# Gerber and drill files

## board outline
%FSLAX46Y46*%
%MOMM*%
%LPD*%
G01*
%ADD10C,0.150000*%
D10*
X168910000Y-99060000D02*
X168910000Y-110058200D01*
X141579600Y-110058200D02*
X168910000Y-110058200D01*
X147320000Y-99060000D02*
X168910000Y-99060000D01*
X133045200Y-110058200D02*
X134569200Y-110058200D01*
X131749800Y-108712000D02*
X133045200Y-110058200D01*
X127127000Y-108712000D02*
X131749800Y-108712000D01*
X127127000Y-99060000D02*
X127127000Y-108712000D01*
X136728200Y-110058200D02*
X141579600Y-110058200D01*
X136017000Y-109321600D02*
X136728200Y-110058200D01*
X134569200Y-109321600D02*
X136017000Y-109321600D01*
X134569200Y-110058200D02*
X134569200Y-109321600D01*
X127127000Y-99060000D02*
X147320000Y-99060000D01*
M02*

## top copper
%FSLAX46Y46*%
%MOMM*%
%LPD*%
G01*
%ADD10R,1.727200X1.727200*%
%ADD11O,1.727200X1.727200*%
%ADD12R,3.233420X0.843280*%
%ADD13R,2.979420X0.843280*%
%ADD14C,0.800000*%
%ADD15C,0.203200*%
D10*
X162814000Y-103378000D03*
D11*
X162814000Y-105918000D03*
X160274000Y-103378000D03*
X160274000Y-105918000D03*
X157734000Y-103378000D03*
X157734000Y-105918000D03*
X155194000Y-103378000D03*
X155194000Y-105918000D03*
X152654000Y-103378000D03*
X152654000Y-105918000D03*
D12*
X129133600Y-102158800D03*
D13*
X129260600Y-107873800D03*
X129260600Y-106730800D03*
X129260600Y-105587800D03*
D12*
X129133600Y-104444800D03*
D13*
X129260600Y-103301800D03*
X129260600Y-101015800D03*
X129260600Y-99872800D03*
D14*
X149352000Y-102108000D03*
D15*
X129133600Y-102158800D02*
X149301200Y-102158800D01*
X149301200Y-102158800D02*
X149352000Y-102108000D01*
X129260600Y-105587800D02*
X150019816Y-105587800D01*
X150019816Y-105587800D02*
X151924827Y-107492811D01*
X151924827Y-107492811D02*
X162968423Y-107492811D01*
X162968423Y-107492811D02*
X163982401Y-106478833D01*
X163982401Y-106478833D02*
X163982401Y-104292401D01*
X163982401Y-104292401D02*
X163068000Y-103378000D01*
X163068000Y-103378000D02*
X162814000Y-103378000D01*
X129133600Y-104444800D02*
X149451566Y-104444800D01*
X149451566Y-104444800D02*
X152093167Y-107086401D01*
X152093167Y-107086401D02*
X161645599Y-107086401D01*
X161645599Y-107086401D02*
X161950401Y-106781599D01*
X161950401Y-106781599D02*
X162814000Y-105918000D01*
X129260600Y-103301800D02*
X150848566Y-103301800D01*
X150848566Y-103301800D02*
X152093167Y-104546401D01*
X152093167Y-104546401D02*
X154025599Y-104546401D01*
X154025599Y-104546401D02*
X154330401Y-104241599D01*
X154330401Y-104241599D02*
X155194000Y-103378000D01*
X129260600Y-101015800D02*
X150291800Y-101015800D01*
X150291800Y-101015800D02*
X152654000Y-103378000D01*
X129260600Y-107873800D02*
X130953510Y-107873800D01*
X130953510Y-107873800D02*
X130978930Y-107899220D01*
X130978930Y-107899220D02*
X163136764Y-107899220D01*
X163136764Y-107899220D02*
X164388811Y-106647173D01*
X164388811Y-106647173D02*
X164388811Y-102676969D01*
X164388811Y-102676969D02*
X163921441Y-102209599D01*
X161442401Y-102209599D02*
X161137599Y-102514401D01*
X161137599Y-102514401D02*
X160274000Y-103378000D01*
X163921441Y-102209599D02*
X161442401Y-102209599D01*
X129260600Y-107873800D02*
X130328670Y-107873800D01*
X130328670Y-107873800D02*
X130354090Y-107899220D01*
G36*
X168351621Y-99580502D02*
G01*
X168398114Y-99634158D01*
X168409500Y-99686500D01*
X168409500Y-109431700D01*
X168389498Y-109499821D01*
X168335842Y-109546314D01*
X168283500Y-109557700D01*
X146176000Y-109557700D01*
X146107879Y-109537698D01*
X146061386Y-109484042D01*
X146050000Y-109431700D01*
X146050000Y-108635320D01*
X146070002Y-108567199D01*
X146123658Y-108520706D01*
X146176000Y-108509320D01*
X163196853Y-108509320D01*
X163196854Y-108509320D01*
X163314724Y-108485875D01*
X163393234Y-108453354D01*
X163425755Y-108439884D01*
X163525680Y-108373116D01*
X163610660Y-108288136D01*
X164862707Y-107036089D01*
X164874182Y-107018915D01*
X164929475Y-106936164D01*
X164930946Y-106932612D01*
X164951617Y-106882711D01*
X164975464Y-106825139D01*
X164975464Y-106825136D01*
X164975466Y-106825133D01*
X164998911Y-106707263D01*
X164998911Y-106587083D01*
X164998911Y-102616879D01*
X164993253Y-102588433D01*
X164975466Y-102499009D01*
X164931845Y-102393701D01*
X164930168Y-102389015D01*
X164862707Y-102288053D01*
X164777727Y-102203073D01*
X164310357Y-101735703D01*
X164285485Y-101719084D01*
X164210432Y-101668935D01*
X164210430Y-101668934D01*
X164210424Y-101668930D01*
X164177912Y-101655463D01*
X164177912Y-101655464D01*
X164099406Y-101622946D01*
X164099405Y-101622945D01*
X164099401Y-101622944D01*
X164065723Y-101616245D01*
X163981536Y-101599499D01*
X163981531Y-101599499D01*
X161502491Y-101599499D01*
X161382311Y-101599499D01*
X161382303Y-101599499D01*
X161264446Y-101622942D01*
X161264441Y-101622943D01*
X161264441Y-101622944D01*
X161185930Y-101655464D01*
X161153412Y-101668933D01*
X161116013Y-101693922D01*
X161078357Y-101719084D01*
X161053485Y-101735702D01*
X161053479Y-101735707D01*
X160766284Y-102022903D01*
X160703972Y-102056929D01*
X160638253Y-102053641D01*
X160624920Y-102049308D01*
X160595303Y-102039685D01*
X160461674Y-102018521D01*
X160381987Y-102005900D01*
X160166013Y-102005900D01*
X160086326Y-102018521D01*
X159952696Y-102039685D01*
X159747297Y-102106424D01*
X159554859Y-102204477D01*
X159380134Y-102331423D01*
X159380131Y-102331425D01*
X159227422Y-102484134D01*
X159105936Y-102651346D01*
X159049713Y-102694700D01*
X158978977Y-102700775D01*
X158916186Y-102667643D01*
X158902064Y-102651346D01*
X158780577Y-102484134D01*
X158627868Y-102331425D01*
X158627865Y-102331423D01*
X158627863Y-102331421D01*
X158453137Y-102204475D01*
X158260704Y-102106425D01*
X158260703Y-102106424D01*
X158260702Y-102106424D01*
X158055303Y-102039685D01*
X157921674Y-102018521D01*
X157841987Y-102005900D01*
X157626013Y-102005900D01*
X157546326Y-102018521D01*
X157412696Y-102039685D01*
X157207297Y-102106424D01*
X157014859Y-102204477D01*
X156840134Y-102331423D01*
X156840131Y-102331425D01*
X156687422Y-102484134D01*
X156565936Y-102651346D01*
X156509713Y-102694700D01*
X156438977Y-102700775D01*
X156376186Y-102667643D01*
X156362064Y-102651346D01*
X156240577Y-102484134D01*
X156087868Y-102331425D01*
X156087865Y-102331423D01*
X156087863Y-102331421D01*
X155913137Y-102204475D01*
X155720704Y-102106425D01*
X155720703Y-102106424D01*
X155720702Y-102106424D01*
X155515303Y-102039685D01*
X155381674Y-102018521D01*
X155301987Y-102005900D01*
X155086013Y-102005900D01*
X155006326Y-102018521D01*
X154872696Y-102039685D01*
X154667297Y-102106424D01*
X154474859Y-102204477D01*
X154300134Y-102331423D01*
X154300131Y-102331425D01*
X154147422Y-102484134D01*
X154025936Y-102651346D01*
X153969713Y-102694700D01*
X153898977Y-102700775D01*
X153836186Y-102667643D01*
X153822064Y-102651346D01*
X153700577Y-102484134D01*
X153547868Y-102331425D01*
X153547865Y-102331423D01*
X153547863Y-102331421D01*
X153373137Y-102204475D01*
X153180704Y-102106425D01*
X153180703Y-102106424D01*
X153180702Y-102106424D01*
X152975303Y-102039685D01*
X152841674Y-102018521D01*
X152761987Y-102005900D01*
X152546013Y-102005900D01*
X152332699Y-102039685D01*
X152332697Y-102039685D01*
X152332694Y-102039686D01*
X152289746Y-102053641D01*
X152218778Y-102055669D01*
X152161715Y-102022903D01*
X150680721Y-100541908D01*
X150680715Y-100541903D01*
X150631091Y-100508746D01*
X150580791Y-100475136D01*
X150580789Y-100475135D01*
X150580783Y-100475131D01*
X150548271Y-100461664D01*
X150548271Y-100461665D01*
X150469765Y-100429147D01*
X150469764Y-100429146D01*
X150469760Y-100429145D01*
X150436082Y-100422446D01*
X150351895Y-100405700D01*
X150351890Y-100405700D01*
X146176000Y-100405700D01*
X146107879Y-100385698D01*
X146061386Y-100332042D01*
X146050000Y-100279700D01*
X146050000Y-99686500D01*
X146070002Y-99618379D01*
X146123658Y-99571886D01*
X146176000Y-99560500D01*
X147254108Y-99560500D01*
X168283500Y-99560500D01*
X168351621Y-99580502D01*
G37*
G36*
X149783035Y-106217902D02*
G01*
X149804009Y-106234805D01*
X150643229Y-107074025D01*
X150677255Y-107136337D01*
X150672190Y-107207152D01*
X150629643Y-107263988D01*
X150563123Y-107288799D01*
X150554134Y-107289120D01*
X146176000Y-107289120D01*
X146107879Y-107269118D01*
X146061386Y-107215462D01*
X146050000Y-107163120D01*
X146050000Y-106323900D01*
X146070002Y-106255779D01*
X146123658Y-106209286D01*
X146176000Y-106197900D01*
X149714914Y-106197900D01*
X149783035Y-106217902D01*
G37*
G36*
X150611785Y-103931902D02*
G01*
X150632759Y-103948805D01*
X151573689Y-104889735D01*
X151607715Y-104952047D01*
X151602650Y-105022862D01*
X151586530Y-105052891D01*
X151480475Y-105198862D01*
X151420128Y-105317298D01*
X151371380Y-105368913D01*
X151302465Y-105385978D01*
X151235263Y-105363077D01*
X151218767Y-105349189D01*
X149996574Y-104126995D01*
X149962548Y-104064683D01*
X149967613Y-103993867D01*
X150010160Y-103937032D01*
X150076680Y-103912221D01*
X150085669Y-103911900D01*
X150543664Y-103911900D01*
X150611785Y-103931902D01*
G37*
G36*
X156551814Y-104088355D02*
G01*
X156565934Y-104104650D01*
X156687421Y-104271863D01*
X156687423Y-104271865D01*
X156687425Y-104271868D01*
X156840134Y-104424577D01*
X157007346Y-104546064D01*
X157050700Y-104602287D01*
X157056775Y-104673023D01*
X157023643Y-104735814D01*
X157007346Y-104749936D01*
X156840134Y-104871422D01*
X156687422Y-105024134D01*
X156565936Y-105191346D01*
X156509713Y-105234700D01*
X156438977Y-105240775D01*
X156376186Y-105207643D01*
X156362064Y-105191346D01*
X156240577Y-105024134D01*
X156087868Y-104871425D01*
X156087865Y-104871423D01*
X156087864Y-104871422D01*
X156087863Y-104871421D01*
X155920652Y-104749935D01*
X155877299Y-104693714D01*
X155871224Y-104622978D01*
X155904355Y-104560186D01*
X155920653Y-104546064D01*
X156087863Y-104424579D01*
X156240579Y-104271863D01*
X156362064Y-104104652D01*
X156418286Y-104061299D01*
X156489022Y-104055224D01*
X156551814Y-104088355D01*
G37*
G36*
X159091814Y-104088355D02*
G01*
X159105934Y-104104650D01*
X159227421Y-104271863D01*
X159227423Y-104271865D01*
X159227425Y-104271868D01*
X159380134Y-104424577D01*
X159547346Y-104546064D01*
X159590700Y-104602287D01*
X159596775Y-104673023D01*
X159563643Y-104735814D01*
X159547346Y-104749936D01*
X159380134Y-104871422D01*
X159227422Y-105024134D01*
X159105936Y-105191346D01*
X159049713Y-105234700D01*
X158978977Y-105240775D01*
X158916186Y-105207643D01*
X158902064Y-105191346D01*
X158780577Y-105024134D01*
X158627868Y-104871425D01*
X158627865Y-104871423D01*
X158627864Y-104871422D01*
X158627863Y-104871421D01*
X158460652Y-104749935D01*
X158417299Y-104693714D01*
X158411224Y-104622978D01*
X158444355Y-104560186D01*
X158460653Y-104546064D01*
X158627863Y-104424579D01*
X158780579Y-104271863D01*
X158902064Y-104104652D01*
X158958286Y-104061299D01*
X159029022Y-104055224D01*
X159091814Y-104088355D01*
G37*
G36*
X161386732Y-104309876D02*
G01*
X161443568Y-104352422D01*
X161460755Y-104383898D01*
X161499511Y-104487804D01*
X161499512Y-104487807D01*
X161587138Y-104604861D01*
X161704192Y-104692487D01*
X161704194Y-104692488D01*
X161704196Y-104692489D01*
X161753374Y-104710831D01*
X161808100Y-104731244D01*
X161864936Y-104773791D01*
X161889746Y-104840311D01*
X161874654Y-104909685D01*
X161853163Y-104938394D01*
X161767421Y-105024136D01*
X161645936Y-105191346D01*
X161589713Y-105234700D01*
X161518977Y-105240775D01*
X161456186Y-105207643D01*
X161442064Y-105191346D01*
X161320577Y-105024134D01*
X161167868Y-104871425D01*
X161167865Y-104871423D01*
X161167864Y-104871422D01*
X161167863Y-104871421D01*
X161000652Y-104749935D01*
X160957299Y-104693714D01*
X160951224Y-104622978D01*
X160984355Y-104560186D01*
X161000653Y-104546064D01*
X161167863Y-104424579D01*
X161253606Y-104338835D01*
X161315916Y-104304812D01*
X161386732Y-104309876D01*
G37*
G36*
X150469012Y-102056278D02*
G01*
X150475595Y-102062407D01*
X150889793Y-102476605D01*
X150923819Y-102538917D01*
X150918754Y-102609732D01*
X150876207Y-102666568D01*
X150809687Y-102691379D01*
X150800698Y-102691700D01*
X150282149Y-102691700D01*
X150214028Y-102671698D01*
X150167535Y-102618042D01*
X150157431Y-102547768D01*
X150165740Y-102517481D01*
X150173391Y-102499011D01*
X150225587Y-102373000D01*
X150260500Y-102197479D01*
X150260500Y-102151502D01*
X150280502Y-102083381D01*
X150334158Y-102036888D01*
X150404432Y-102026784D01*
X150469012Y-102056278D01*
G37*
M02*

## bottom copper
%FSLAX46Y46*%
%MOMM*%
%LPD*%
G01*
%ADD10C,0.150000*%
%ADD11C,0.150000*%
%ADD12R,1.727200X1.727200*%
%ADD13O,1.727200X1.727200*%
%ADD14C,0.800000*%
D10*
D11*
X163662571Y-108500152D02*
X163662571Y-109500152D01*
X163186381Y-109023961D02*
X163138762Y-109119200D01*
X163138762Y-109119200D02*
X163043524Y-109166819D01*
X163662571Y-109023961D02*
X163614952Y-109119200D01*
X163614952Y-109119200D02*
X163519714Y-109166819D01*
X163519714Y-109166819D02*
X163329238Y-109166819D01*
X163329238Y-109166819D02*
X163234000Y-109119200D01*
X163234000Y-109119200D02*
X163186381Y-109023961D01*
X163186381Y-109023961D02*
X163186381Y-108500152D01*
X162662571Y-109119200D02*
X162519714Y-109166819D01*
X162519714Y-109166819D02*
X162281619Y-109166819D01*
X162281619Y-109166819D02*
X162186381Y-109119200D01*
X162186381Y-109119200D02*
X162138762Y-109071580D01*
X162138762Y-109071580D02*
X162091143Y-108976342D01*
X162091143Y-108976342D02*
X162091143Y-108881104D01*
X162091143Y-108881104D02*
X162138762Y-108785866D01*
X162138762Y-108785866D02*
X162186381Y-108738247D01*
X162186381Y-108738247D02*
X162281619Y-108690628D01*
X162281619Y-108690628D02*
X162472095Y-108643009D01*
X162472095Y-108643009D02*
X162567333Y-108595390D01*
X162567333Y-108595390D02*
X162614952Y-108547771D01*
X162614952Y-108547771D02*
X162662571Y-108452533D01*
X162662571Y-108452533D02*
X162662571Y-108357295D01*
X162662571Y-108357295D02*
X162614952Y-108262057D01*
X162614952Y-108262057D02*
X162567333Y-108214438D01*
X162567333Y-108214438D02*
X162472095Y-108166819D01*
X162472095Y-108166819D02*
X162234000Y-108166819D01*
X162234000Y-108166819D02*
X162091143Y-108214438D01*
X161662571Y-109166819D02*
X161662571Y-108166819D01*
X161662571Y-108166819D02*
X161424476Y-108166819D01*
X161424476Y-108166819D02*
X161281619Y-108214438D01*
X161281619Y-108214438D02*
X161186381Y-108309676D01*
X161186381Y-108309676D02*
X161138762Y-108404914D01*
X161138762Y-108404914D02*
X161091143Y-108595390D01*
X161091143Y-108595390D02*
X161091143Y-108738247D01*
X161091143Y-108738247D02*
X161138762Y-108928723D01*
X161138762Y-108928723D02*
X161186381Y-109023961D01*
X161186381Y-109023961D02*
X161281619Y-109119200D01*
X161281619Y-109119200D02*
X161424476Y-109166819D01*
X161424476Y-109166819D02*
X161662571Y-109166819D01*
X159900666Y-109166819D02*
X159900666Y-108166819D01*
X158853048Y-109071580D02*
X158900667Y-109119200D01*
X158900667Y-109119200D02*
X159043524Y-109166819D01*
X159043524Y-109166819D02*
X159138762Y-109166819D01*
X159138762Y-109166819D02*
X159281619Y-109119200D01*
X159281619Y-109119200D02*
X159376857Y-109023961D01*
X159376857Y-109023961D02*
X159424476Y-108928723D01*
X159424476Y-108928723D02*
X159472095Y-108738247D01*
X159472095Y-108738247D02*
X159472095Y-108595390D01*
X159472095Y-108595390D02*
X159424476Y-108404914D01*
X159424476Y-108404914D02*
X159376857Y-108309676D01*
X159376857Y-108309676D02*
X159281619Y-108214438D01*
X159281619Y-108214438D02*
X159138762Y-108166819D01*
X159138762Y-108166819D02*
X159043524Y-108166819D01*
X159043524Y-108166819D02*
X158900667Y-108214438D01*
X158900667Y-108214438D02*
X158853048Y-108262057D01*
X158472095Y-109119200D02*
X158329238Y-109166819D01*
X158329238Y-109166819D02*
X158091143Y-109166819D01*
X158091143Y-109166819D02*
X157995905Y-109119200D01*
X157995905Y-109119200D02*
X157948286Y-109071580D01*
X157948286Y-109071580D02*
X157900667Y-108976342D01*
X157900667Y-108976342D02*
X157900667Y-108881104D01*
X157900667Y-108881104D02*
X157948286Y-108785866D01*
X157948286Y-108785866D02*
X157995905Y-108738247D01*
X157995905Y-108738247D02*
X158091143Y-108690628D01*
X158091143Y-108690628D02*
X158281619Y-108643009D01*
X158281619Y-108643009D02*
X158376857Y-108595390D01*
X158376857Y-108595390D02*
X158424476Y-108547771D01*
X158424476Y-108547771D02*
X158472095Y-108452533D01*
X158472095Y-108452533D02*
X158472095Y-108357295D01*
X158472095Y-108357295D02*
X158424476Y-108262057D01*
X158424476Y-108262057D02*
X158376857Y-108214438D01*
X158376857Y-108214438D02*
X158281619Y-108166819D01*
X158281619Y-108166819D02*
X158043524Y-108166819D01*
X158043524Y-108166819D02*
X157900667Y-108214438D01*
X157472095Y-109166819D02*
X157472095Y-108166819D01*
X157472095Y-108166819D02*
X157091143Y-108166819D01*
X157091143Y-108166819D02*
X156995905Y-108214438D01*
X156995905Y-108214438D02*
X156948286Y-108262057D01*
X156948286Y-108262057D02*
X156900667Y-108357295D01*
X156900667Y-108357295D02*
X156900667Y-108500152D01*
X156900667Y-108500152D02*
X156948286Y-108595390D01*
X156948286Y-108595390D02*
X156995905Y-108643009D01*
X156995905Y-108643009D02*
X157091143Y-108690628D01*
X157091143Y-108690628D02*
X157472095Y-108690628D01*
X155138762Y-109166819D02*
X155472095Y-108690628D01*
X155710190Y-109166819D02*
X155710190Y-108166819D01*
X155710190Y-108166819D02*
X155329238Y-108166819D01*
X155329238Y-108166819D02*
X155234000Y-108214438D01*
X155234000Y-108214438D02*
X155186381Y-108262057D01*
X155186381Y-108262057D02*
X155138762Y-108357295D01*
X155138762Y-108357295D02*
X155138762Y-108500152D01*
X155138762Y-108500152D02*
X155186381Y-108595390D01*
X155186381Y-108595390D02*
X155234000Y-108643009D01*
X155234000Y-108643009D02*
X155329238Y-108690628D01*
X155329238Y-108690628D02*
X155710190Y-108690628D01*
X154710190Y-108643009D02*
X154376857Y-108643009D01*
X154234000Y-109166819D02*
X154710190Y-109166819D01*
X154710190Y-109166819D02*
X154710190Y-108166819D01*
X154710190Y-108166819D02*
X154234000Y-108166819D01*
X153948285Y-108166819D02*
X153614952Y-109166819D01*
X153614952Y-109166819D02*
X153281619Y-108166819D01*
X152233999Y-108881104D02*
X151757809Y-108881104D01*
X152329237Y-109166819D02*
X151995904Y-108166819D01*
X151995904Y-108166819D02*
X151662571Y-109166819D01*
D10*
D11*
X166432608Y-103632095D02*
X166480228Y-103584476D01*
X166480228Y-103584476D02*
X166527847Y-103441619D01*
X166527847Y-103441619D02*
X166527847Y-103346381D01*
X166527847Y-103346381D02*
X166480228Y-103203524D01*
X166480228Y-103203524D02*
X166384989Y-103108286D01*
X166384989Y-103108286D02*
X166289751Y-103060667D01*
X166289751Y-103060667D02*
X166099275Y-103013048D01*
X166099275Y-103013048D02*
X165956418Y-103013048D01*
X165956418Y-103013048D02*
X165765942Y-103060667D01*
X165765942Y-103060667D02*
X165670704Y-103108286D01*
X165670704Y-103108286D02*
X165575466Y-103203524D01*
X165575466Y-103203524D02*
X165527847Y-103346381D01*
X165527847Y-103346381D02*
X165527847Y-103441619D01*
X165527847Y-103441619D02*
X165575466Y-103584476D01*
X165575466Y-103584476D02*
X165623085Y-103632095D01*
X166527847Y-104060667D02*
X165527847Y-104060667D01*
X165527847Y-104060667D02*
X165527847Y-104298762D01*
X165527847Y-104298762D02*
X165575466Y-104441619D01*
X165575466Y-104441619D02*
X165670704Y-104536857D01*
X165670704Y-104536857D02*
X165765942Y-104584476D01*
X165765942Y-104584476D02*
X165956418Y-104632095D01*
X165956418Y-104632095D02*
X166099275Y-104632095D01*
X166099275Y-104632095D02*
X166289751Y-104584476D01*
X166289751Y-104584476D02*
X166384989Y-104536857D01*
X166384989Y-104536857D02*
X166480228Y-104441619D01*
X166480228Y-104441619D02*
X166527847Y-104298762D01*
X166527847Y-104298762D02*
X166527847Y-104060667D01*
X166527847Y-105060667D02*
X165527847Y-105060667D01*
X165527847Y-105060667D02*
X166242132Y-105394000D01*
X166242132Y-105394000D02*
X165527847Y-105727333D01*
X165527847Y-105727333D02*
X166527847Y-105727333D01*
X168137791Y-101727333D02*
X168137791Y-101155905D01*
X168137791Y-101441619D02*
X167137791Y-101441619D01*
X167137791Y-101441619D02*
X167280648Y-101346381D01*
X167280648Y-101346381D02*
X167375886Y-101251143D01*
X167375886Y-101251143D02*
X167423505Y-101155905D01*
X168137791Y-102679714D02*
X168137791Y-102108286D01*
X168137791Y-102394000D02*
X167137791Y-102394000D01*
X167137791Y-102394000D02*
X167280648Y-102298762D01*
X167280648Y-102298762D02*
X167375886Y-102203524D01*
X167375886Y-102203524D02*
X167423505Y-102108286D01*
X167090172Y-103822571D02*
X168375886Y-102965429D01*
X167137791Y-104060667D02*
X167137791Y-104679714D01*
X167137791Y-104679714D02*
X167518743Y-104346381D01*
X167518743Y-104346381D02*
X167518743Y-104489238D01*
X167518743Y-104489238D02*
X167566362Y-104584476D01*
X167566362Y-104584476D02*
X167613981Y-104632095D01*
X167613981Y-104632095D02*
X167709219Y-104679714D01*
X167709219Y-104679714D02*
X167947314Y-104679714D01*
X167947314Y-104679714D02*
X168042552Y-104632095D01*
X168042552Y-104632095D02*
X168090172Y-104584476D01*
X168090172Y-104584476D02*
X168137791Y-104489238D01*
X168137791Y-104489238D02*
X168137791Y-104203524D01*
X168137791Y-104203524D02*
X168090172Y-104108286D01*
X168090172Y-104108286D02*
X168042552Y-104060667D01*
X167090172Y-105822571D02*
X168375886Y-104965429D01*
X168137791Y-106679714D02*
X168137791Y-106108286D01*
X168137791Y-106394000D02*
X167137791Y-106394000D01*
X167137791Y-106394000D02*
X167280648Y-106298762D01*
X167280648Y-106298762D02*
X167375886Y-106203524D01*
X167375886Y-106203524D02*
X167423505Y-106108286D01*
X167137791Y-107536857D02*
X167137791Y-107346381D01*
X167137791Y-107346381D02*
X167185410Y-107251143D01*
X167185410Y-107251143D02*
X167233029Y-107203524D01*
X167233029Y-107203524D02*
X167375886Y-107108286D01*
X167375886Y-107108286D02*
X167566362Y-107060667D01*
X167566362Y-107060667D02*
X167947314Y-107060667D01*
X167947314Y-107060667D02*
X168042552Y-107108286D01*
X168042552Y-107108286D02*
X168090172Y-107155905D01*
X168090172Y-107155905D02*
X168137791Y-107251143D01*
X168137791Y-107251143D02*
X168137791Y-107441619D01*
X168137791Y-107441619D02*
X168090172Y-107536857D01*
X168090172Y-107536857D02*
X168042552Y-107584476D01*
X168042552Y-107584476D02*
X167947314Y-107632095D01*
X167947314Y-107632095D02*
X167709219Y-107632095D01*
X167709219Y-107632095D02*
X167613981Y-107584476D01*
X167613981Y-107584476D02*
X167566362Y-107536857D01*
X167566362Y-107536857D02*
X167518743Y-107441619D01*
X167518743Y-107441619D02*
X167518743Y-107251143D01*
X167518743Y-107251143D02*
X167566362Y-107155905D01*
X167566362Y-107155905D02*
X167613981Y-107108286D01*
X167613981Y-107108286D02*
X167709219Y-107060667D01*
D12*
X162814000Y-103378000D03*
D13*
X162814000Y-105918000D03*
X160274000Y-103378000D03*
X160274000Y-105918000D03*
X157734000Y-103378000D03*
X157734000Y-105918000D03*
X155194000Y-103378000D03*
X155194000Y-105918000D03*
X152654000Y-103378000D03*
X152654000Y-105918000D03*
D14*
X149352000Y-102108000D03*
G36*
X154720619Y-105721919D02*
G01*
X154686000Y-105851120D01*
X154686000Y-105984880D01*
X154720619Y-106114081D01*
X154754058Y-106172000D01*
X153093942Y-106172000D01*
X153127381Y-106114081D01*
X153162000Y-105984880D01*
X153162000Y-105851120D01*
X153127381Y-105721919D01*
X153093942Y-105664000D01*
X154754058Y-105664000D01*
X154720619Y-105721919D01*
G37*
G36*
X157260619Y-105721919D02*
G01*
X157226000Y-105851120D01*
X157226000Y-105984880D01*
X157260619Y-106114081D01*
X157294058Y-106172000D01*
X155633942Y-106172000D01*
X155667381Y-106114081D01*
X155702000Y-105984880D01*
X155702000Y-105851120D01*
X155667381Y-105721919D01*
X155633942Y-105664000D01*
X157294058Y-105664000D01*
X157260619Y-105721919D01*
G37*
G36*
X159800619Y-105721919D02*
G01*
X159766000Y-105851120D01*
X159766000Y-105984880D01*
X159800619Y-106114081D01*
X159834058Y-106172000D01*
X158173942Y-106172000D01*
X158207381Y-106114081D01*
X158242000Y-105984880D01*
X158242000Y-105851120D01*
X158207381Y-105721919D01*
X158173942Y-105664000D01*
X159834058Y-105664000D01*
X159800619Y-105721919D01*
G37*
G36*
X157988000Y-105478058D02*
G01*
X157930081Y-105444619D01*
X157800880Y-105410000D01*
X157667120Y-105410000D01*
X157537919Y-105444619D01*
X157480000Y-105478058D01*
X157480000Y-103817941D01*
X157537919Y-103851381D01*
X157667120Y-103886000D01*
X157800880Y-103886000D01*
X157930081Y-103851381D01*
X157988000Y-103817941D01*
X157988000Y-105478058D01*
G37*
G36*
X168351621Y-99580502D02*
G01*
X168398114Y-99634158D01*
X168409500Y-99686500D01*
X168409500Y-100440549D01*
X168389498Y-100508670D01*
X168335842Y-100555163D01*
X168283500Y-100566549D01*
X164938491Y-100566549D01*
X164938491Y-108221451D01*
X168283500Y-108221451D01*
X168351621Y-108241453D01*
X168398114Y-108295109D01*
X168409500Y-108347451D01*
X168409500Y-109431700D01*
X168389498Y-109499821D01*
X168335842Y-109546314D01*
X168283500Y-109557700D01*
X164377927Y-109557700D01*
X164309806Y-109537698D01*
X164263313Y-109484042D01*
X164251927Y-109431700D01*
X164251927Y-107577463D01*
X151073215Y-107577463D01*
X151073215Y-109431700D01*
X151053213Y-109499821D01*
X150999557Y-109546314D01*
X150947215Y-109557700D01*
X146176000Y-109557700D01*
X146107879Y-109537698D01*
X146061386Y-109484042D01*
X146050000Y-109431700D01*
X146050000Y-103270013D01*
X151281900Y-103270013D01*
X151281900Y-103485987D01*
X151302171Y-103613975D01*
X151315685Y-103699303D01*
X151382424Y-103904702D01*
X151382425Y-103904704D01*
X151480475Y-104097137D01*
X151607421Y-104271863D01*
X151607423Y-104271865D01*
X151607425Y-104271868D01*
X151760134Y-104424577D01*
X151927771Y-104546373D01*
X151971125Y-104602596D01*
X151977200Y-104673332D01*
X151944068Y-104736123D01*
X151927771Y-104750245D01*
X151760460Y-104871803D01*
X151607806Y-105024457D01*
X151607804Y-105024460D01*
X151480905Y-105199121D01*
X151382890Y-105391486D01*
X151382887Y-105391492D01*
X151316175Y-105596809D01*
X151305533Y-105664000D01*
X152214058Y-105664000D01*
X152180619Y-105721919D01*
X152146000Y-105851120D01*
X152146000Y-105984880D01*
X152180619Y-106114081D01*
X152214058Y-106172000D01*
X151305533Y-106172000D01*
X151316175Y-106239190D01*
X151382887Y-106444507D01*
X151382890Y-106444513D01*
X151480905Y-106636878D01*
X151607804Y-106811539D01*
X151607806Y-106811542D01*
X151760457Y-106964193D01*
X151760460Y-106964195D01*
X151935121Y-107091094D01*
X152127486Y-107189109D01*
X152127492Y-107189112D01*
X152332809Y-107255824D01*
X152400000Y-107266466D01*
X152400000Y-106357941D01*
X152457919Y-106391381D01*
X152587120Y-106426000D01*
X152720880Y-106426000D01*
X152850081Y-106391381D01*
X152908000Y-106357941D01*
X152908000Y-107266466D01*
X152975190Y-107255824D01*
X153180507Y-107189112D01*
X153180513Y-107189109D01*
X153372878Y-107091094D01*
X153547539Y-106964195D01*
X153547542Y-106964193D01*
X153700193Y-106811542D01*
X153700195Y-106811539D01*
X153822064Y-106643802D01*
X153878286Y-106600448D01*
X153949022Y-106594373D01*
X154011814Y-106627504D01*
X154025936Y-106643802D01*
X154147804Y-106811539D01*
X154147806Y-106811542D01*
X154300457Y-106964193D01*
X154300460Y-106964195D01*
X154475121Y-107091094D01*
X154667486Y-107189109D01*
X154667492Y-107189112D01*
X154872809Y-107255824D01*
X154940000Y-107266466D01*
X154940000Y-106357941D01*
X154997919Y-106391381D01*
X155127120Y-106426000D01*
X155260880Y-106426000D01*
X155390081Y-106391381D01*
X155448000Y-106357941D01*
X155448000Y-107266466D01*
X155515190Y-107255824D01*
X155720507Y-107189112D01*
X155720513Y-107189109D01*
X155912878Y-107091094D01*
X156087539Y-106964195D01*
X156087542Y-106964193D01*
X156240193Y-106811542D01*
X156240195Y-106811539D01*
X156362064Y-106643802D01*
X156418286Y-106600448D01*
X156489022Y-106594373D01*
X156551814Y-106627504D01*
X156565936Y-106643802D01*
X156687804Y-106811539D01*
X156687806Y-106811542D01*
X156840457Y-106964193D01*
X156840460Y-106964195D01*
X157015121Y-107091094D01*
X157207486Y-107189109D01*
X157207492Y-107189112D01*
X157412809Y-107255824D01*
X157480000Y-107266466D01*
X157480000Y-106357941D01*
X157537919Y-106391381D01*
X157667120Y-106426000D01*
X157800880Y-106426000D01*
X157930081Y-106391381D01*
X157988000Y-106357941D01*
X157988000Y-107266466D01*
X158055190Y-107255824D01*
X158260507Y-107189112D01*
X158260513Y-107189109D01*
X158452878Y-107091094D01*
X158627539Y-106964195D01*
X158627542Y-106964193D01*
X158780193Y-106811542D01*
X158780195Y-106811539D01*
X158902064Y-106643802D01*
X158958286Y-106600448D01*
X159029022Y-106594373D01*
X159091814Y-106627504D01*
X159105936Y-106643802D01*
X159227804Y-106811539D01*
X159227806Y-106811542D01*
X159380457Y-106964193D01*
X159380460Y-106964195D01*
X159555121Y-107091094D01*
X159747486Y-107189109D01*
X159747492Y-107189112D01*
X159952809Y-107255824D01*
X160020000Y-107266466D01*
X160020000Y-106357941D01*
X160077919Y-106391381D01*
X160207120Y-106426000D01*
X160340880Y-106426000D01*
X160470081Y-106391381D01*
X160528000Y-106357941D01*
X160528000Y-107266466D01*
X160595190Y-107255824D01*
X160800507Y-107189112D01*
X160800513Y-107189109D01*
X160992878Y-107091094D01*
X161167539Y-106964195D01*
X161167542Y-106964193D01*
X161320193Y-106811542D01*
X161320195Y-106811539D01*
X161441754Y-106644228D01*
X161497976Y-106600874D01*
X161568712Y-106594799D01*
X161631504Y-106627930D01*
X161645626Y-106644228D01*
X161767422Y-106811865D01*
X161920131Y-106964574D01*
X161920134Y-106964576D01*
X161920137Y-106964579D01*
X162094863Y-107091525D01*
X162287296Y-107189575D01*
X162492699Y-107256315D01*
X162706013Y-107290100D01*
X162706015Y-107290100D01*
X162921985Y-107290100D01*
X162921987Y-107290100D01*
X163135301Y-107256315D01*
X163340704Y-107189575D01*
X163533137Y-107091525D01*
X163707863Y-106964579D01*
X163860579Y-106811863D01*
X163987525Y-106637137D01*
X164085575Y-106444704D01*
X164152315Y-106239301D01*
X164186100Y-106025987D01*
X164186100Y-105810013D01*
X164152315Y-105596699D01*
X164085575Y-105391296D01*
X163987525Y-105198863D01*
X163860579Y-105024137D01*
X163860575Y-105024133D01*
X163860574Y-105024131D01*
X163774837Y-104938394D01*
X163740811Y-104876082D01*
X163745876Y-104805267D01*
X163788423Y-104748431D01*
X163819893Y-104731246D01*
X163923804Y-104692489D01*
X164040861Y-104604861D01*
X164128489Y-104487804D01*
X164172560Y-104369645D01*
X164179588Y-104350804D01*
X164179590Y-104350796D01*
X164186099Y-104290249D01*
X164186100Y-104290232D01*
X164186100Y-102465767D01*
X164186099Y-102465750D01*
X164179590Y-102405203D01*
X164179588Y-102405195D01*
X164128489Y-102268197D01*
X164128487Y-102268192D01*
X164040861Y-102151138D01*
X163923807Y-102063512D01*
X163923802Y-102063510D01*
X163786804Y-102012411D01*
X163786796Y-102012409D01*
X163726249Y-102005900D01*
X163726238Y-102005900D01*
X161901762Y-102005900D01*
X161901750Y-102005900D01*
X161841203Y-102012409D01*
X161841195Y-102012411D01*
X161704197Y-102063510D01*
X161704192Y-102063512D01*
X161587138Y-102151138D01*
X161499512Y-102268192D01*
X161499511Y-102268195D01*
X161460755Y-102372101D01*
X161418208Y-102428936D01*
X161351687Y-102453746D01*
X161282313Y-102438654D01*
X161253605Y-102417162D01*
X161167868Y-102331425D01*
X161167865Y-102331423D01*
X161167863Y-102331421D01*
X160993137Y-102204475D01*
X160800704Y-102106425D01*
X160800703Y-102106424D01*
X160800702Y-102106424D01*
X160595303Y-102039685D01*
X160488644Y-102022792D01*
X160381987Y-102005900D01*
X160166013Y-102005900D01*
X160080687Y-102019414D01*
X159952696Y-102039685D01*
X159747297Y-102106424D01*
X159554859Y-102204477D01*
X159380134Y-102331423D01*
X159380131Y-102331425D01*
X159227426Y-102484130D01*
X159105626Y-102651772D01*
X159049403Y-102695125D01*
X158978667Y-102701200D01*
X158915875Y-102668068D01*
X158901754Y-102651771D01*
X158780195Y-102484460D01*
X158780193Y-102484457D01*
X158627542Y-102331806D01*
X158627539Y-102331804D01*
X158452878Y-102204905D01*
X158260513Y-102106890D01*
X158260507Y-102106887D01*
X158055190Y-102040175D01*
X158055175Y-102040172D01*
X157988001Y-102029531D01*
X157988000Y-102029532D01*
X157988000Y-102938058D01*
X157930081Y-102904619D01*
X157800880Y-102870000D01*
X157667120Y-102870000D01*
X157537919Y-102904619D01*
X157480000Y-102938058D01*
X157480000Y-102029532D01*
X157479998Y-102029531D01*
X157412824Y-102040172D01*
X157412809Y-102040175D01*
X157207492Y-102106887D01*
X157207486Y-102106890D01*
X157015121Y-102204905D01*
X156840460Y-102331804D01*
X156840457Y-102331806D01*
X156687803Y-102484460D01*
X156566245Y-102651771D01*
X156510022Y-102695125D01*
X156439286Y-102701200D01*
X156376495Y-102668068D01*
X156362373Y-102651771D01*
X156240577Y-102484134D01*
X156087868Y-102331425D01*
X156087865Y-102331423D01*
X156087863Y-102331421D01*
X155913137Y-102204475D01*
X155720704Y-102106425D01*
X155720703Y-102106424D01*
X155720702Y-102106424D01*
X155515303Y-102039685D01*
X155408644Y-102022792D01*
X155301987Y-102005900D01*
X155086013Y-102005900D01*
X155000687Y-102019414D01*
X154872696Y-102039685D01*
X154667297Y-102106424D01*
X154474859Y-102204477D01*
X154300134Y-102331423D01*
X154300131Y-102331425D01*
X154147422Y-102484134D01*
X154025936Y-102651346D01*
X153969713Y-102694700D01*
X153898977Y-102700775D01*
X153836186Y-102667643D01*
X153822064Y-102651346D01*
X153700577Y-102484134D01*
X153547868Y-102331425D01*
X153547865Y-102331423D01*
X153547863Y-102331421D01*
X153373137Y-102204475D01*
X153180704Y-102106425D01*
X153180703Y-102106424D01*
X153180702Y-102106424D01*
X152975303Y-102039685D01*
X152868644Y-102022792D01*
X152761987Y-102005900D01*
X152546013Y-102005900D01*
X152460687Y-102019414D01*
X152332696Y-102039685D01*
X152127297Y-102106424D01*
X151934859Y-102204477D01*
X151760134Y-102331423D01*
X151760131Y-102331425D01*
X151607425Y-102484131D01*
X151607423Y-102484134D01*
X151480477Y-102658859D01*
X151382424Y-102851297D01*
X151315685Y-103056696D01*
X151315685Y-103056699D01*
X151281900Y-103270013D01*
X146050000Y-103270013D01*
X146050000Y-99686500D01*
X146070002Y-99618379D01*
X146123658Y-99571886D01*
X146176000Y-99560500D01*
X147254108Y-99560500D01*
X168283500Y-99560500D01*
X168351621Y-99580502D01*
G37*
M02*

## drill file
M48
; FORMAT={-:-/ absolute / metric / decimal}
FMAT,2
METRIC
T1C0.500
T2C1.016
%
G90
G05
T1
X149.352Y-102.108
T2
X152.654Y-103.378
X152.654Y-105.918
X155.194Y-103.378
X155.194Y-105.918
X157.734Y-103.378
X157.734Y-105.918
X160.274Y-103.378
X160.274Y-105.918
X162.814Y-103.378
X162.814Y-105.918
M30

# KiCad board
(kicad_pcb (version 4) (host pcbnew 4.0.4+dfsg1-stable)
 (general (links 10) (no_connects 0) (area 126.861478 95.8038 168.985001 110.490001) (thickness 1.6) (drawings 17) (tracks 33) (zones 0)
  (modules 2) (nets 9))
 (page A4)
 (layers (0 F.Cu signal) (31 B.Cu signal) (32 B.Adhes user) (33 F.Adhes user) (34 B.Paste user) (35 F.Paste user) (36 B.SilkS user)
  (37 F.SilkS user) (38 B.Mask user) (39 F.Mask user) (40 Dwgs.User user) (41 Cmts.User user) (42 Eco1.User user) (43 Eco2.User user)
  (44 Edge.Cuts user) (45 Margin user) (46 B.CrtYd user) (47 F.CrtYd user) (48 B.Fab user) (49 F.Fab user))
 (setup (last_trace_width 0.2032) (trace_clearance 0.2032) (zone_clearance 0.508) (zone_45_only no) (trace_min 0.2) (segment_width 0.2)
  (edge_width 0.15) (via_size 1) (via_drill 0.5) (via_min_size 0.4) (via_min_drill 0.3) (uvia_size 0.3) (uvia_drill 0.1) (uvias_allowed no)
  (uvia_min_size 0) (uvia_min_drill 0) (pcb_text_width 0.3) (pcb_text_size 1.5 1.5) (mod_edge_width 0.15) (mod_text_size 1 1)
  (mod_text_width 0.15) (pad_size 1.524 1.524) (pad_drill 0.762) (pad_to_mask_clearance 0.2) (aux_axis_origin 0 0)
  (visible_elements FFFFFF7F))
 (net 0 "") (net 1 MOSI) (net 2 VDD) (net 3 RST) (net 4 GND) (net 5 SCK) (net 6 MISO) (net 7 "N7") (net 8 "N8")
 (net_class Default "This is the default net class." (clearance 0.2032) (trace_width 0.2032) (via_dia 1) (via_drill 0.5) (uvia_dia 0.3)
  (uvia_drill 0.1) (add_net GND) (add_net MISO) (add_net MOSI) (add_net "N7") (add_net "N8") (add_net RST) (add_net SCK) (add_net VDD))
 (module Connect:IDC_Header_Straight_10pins (layer F.Cu) (at 162.814 103.378 180)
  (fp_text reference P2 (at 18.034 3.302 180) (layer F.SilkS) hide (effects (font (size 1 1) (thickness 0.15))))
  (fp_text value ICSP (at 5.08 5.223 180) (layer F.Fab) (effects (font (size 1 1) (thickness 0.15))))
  (pad 1 thru_hole rect (at 0 0 180) (size 1.7272 1.7272) (drill 1.016) (layers *.Cu *.Mask F.SilkS) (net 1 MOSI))
  (pad 2 thru_hole oval (at 0 -2.54 180) (size 1.7272 1.7272) (drill 1.016) (layers *.Cu *.Mask F.SilkS) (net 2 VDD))
  (pad 3 thru_hole oval (at 2.54 0 180) (size 1.7272 1.7272) (drill 1.016) (layers *.Cu *.Mask F.SilkS) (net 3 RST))
  (pad 4 thru_hole oval (at 2.54 -2.54 180) (size 1.7272 1.7272) (drill 1.016) (layers *.Cu *.Mask F.SilkS) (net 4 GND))
  (pad 5 thru_hole oval (at 5.08 0 180) (size 1.7272 1.7272) (drill 1.016) (layers *.Cu *.Mask F.SilkS) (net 4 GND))
  (pad 6 thru_hole oval (at 5.08 -2.54 180) (size 1.7272 1.7272) (drill 1.016) (layers *.Cu *.Mask F.SilkS) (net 4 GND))
  (pad 7 thru_hole oval (at 7.62 0 180) (size 1.7272 1.7272) (drill 1.016) (layers *.Cu *.Mask F.SilkS) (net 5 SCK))
  (pad 8 thru_hole oval (at 7.62 -2.54 180) (size 1.7272 1.7272) (drill 1.016) (layers *.Cu *.Mask F.SilkS) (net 4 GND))
  (pad 9 thru_hole oval (at 10.16 0 180) (size 1.7272 1.7272) (drill 1.016) (layers *.Cu *.Mask F.SilkS) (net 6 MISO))
  (pad 10 thru_hole oval (at 10.16 -2.54 180) (size 1.7272 1.7272) (drill 1.016) (layers *.Cu *.Mask F.SilkS) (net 4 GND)))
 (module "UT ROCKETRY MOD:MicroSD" (layer F.Cu) (at 134.874 97.282)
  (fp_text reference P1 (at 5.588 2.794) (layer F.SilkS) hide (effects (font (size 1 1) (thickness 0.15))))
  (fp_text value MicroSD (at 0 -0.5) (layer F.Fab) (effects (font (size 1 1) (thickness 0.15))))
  (pad 6 smd rect (at -5.7404 4.8768) (size 3.23342 0.84328) (layers F.Cu F.Paste F.Mask) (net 4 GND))
  (pad 1 smd rect (at -5.6134 10.5918) (size 2.97942 0.84328) (layers F.Cu F.Paste F.Mask) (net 3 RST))
  (pad 2 smd rect (at -5.6134 9.4488) (size 2.97942 0.84328) (layers F.Cu F.Paste F.Mask) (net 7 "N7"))
  (pad 3 smd rect (at -5.6134 8.3058) (size 2.97942 0.84328) (layers F.Cu F.Paste F.Mask) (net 1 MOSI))
  (pad 4 smd rect (at -5.7404 7.1628) (size 3.23342 0.84328) (layers F.Cu F.Paste F.Mask) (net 2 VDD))
  (pad 5 smd rect (at -5.6134 6.0198) (size 2.97942 0.84328) (layers F.Cu F.Paste F.Mask) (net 5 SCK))
  (pad 7 smd rect (at -5.6134 3.7338) (size 2.97942 0.84328) (layers F.Cu F.Paste F.Mask) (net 6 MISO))
  (pad 8 smd rect (at -5.6134 2.5908) (size 2.97942 0.84328) (layers F.Cu F.Paste F.Mask) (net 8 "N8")))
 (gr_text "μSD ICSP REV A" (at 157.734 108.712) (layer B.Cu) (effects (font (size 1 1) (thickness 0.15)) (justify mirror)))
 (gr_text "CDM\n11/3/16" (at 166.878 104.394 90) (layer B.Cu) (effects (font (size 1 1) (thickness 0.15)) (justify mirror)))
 (gr_line (start 168.91 99.06) (end 168.91 110.0582) (layer Edge.Cuts) (width 0.15))
 (gr_line (start 141.5796 110.0582) (end 168.91 110.0582) (layer Edge.Cuts) (width 0.15))
 (gr_line (start 147.32 99.06) (end 168.91 99.06) (layer Edge.Cuts) (width 0.15))
 (gr_line (start 133.0452 110.0582) (end 134.5692 110.0582) (layer Edge.Cuts) (width 0.15))
 (gr_line (start 131.7498 108.712) (end 133.0452 110.0582) (layer Edge.Cuts) (width 0.15))
 (gr_line (start 127.127 108.712) (end 131.7498 108.712) (layer Edge.Cuts) (width 0.15))
 (gr_line (start 127.127 99.06) (end 127.127 108.712) (layer Edge.Cuts) (width 0.15))
 (gr_line (start 136.7282 110.0582) (end 141.5796 110.0582) (layer Edge.Cuts) (width 0.15))
 (gr_line (start 136.017 109.3216) (end 136.7282 110.0582) (layer Edge.Cuts) (width 0.15))
 (gr_line (start 134.5692 109.3216) (end 136.017 109.3216) (layer Edge.Cuts) (width 0.15))
 (gr_line (start 134.5692 110.0582) (end 134.5692 109.3216) (layer Edge.Cuts) (width 0.15))
 (gr_line (start 127.127 99.06) (end 147.32 99.06) (layer Edge.Cuts) (width 0.15))
 (segment (start 129.1336 102.1588) (end 149.3012 102.1588) (width 0.2032) (layer F.Cu) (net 4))
 (segment (start 149.3012 102.1588) (end 149.352 102.108) (width 0.2032) (layer F.Cu) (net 4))
 (via (at 149.352 102.108) (size 0.8) (drill 0.5) (layers F.Cu B.Cu) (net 4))
 (segment (start 129.2606 105.5878) (end 150.019816 105.5878) (width 0.2032) (layer F.Cu) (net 1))
 (segment (start 150.019816 105.5878) (end 151.924827 107.492811) (width 0.2032) (layer F.Cu) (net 1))
 (segment (start 151.924827 107.492811) (end 162.968423 107.492811) (width 0.2032) (layer F.Cu) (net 1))
 (segment (start 162.968423 107.492811) (end 163.982401 106.478833) (width 0.2032) (layer F.Cu) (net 1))
 (segment (start 163.982401 106.478833) (end 163.982401 104.292401) (width 0.2032) (layer F.Cu) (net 1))
 (segment (start 163.982401 104.292401) (end 163.068 103.378) (width 0.2032) (layer F.Cu) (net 1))
 (segment (start 163.068 103.378) (end 162.814 103.378) (width 0.2032) (layer F.Cu) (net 1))
 (segment (start 129.1336 104.4448) (end 149.451566 104.4448) (width 0.2032) (layer F.Cu) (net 2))
 (segment (start 149.451566 104.4448) (end 152.093167 107.086401) (width 0.2032) (layer F.Cu) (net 2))
 (segment (start 152.093167 107.086401) (end 161.645599 107.086401) (width 0.2032) (layer F.Cu) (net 2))
 (segment (start 161.645599 107.086401) (end 161.950401 106.781599) (width 0.2032) (layer F.Cu) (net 2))
 (segment (start 161.950401 106.781599) (end 162.814 105.918) (width 0.2032) (layer F.Cu) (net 2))
 (segment (start 129.2606 103.3018) (end 150.848566 103.3018) (width 0.2032) (layer F.Cu) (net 5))
 (segment (start 150.848566 103.3018) (end 152.093167 104.546401) (width 0.2032) (layer F.Cu) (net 5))
 (segment (start 152.093167 104.546401) (end 154.025599 104.546401) (width 0.2032) (layer F.Cu) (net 5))
 (segment (start 154.025599 104.546401) (end 154.330401 104.241599) (width 0.2032) (layer F.Cu) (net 5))
 (segment (start 154.330401 104.241599) (end 155.194 103.378) (width 0.2032) (layer F.Cu) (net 5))
 (segment (start 129.2606 101.0158) (end 150.2918 101.0158) (width 0.2032) (layer F.Cu) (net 6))
 (segment (start 150.2918 101.0158) (end 152.654 103.378) (width 0.2032) (layer F.Cu) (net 6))
 (segment (start 129.2606 107.8738) (end 130.95351 107.8738) (width 0.2032) (layer F.Cu) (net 3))
 (segment (start 130.95351 107.8738) (end 130.97893 107.89922) (width 0.2032) (layer F.Cu) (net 3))
 (segment (start 130.97893 107.89922) (end 163.136764 107.89922) (width 0.2032) (layer F.Cu) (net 3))
 (segment (start 163.136764 107.89922) (end 164.388811 106.647173) (width 0.2032) (layer F.Cu) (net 3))
 (segment (start 164.388811 106.647173) (end 164.388811 102.676969) (width 0.2032) (layer F.Cu) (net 3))
 (segment (start 164.388811 102.676969) (end 163.921441 102.209599) (width 0.2032) (layer F.Cu) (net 3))
 (segment (start 161.442401 102.209599) (end 161.137599 102.514401) (width 0.2032) (layer F.Cu) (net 3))
 (segment (start 161.137599 102.514401) (end 160.274 103.378) (width 0.2032) (layer F.Cu) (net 3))
 (segment (start 163.921441 102.209599) (end 161.442401 102.209599) (width 0.2032) (layer F.Cu) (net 3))
 (segment (start 129.2606 107.8738) (end 130.32867 107.8738) (width 0.2032) (layer F.Cu) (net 3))
 (segment (start 130.32867 107.8738) (end 130.35409 107.89922) (width 0.2032) (layer F.Cu) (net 3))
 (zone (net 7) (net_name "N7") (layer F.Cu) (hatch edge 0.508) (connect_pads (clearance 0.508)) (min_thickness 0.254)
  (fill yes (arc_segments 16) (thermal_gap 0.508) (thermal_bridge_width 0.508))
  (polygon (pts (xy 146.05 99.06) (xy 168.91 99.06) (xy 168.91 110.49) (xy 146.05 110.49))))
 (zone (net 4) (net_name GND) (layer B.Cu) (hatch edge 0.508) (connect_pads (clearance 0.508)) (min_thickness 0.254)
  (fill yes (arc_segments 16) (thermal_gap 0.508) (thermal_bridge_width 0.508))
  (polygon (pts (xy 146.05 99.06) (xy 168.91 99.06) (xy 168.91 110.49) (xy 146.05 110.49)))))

